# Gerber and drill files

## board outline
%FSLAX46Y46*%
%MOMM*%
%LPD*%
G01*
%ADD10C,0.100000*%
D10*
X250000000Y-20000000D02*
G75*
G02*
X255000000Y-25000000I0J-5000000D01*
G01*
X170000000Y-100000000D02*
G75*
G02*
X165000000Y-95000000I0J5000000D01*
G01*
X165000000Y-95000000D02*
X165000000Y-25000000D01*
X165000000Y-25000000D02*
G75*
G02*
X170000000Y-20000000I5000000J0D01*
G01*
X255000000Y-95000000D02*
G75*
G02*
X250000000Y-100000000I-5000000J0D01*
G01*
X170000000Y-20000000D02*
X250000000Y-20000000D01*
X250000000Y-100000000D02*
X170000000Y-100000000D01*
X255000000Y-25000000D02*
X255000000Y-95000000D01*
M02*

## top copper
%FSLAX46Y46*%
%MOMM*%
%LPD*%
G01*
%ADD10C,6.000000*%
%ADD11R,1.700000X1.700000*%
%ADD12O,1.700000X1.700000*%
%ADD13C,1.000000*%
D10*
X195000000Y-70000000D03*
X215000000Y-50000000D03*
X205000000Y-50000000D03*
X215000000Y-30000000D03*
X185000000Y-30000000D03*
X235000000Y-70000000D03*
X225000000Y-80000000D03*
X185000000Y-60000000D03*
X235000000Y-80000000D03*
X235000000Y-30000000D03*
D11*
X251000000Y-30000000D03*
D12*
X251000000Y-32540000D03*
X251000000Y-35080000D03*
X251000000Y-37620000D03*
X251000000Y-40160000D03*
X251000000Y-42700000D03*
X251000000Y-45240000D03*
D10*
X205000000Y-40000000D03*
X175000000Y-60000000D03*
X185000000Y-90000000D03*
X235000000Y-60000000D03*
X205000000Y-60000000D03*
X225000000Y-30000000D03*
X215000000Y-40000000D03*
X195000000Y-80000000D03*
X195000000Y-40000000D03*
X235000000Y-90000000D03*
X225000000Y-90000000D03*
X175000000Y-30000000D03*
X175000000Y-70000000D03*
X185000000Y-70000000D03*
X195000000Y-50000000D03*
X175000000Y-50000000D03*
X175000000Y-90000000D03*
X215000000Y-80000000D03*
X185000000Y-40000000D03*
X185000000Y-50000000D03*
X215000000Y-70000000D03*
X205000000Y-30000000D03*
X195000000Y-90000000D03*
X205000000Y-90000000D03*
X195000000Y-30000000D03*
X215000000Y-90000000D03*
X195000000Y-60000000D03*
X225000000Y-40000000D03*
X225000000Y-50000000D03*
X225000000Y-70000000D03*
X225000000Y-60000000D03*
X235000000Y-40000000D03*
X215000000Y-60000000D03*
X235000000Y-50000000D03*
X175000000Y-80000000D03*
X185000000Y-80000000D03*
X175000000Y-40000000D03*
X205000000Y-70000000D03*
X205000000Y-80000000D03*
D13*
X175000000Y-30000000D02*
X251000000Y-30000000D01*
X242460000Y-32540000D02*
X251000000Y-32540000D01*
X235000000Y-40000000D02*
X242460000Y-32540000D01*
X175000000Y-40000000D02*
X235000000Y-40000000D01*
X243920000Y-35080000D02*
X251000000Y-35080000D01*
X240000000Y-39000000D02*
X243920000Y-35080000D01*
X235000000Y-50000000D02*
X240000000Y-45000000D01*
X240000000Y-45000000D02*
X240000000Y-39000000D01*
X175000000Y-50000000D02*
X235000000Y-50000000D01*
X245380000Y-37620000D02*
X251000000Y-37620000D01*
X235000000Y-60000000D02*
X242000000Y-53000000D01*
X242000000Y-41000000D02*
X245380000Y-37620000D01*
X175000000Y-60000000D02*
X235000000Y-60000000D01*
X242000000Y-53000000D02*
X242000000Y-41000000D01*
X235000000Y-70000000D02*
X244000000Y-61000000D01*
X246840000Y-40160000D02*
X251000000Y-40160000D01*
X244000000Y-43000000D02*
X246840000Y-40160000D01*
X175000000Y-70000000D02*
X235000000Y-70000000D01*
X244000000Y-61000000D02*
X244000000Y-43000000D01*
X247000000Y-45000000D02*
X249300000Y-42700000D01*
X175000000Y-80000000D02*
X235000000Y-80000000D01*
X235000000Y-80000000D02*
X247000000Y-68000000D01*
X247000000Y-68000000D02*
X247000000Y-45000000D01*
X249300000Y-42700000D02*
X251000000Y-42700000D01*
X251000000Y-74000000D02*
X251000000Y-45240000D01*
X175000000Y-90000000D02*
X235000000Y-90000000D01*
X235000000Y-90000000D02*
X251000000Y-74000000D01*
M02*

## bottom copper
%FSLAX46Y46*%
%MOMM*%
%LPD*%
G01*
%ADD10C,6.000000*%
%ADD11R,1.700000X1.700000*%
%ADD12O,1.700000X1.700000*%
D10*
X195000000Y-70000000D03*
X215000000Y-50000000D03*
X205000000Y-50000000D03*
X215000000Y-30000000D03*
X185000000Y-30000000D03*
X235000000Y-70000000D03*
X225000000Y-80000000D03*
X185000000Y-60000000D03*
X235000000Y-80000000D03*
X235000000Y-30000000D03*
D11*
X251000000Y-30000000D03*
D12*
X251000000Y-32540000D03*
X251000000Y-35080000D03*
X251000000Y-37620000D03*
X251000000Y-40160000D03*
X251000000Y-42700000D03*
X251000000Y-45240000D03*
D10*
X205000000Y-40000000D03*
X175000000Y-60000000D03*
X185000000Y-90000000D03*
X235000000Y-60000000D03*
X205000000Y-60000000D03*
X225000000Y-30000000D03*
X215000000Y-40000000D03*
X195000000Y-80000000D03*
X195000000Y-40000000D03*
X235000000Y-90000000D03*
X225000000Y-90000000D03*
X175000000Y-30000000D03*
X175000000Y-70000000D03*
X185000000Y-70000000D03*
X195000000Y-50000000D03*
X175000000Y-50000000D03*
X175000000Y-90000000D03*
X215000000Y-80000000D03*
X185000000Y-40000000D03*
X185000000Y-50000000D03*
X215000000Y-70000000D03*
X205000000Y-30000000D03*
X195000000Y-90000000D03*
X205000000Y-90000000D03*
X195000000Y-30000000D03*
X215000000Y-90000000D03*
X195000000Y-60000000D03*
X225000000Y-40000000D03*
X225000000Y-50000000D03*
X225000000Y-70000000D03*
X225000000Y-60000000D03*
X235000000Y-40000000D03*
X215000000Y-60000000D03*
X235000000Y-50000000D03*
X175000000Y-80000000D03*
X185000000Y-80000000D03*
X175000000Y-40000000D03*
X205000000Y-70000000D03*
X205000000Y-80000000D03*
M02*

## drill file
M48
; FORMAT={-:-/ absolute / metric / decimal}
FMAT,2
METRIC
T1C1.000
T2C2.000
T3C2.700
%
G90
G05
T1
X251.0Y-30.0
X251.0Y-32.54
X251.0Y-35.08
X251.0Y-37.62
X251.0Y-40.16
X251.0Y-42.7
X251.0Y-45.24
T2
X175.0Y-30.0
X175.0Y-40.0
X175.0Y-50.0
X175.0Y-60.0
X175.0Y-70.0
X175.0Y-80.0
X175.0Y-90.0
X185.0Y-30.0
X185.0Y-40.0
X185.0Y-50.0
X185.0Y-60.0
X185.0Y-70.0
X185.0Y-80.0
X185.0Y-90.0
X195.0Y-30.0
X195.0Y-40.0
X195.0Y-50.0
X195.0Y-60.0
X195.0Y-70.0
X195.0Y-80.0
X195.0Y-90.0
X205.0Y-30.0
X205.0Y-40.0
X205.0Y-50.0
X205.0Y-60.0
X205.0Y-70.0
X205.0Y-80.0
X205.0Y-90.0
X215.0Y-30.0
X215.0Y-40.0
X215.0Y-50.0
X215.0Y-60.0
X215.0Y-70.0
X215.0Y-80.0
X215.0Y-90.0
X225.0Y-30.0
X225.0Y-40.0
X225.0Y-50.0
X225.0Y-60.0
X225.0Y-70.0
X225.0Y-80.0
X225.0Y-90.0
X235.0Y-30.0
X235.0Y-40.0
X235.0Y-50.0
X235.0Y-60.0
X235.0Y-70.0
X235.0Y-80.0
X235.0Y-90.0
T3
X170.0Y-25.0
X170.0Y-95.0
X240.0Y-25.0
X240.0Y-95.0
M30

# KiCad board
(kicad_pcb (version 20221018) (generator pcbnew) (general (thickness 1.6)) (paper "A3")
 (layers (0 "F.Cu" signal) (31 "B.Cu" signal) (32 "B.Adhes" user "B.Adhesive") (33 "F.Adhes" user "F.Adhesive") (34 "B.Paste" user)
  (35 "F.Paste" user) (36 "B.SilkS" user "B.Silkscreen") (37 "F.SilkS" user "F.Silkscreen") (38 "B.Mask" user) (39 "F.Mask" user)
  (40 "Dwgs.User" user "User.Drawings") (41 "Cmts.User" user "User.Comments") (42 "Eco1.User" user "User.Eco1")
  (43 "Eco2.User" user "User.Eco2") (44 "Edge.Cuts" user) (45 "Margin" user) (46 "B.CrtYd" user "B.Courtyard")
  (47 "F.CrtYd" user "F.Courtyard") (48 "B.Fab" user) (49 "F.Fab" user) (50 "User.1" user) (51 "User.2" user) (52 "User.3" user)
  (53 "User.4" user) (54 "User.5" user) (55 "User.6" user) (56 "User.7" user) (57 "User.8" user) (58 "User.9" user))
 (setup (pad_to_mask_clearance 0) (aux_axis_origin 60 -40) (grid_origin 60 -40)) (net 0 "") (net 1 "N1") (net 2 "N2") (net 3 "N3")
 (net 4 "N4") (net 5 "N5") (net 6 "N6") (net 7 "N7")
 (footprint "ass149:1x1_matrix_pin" (layer "F.Cu") (at 195 72.54)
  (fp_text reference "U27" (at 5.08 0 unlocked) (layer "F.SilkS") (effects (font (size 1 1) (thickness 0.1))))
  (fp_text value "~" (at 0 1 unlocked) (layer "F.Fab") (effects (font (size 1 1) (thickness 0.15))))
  (pad "1" thru_hole circle (at 0 -2.54) (size 6 6) (drill 2) (layers "*.Cu" "*.Mask") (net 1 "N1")))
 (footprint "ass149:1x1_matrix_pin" (layer "F.Cu") (at 215 47.46 180)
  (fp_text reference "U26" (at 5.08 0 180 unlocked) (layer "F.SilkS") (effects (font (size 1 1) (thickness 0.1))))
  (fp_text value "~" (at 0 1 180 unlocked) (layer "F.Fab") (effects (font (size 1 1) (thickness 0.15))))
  (pad "1" thru_hole circle (at 0 -2.54 180) (size 6 6) (drill 2) (layers "*.Cu" "*.Mask") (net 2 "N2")))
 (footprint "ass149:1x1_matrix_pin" (layer "F.Cu") (at 207.54 50 90)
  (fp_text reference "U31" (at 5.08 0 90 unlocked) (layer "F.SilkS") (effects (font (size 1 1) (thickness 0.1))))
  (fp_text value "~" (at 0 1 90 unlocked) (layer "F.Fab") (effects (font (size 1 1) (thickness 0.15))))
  (pad "1" thru_hole circle (at 0 -2.54 90) (size 6 6) (drill 2) (layers "*.Cu" "*.Mask") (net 2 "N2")))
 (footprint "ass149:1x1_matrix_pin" (layer "F.Cu") (at 217.54 30 90)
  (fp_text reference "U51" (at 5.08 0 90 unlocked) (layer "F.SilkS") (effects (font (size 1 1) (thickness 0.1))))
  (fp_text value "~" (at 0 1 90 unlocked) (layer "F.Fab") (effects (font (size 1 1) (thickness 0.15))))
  (pad "1" thru_hole circle (at 0 -2.54 90) (size 6 6) (drill 2) (layers "*.Cu" "*.Mask") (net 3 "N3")))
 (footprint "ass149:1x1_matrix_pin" (layer "F.Cu") (at 187.54 30 90)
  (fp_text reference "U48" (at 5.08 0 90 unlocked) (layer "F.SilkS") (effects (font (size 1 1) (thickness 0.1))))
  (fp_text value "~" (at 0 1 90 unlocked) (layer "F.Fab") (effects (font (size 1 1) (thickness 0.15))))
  (pad "1" thru_hole circle (at 0 -2.54 90) (size 6 6) (drill 2) (layers "*.Cu" "*.Mask") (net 3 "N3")))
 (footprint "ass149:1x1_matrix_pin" (layer "F.Cu") (at 232.46 70 -90)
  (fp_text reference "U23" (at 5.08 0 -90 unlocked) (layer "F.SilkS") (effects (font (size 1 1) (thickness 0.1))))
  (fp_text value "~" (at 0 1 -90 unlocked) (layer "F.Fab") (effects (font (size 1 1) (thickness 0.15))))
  (pad "1" thru_hole circle (at 0 -2.54 270) (size 6 6) (drill 2) (layers "*.Cu" "*.Mask") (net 1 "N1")))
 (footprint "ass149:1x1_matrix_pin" (layer "F.Cu") (at 227.54 80 90)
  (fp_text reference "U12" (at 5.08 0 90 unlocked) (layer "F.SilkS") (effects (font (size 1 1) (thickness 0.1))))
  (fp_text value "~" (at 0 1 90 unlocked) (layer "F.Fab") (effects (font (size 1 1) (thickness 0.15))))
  (pad "1" thru_hole circle (at 0 -2.54 90) (size 6 6) (drill 2) (layers "*.Cu" "*.Mask") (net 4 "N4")))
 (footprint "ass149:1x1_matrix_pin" (layer "F.Cu") (at 187.54 60 90)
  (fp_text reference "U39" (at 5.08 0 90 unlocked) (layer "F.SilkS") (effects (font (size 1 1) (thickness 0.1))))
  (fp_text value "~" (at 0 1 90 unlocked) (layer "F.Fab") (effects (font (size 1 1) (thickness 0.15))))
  (pad "1" thru_hole circle (at 0 -2.54 90) (size 6 6) (drill 2) (layers "*.Cu" "*.Mask") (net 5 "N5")))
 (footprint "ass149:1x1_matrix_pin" (layer "F.Cu") (at 235 77.46 180)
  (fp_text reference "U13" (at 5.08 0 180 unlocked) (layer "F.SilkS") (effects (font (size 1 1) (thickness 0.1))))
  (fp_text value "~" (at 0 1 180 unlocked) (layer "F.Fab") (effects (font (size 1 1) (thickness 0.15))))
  (pad "1" thru_hole circle (at 0 -2.54 180) (size 6 6) (drill 2) (layers "*.Cu" "*.Mask") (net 4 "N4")))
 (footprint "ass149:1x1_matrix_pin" (layer "F.Cu") (at 237.54 30 90)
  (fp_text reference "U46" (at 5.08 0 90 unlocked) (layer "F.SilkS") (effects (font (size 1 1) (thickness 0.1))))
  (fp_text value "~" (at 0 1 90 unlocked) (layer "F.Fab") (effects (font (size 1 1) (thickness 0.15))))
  (pad "1" thru_hole circle (at 0 -2.54 90) (size 6 6) (drill 2) (layers "*.Cu" "*.Mask") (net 3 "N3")))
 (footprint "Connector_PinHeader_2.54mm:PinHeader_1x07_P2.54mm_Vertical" (layer "F.Cu") (at 251 30)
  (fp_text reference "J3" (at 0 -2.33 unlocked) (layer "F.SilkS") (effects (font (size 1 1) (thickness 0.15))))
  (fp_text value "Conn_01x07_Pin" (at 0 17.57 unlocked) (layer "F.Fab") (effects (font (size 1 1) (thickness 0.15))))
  (pad "1" thru_hole rect (at 0 0) (size 1.7 1.7) (drill 1) (layers "*.Cu" "*.Mask") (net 3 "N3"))
  (pad "2" thru_hole oval (at 0 2.54) (size 1.7 1.7) (drill 1) (layers "*.Cu" "*.Mask") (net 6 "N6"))
  (pad "3" thru_hole oval (at 0 5.08) (size 1.7 1.7) (drill 1) (layers "*.Cu" "*.Mask") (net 2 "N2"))
  (pad "4" thru_hole oval (at 0 7.62) (size 1.7 1.7) (drill 1) (layers "*.Cu" "*.Mask") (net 5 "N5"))
  (pad "5" thru_hole oval (at 0 10.16) (size 1.7 1.7) (drill 1) (layers "*.Cu" "*.Mask") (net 1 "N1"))
  (pad "6" thru_hole oval (at 0 12.7) (size 1.7 1.7) (drill 1) (layers "*.Cu" "*.Mask") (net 4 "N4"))
  (pad "7" thru_hole oval (at 0 15.24) (size 1.7 1.7) (drill 1) (layers "*.Cu" "*.Mask") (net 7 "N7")))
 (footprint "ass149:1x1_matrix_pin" (layer "F.Cu") (at 207.54 40 90)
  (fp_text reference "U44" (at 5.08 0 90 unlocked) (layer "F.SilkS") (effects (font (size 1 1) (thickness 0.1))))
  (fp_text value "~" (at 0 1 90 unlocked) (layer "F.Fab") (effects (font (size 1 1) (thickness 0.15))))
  (pad "1" thru_hole circle (at 0 -2.54 90) (size 6 6) (drill 2) (layers "*.Cu" "*.Mask") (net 6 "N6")))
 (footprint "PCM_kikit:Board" (layer "F.Cu") (at 236.5 100 180)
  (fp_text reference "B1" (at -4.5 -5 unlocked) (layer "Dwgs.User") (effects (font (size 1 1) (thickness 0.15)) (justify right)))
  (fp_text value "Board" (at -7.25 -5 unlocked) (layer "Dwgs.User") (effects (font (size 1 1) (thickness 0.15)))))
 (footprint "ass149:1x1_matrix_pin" (layer "F.Cu") (at 175 57.46 180)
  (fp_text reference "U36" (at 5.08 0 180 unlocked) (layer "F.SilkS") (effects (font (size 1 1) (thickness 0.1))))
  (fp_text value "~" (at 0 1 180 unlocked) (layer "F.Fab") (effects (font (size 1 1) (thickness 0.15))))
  (pad "1" thru_hole circle (at 0 -2.54 180) (size 6 6) (drill 2) (layers "*.Cu" "*.Mask") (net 5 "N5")))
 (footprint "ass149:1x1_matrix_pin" (layer "F.Cu") (at 187.54 90 90)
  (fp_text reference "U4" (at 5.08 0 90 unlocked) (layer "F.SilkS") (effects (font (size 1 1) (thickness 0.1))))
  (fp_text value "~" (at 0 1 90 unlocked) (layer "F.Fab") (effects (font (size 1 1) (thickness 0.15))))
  (pad "1" thru_hole circle (at 0 -2.54 90) (size 6 6) (drill 2) (layers "*.Cu" "*.Mask") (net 7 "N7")))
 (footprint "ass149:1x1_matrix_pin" (layer "F.Cu") (at 235 57.46 180)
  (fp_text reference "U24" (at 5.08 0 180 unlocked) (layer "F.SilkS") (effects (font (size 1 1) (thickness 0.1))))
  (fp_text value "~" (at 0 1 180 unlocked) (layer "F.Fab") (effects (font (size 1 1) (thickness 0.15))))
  (pad "1" thru_hole circle (at 0 -2.54 180) (size 6 6) (drill 2) (layers "*.Cu" "*.Mask") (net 5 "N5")))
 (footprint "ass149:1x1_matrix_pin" (layer "F.Cu") (at 207.54 60 90)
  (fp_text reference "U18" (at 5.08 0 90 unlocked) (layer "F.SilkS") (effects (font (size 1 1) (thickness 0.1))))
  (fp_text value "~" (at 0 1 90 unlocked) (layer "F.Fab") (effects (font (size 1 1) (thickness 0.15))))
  (pad "1" thru_hole circle (at 0 -2.54 90) (size 6 6) (drill 2) (layers "*.Cu" "*.Mask") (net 5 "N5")))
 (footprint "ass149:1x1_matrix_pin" (layer "F.Cu") (at 225 32.54)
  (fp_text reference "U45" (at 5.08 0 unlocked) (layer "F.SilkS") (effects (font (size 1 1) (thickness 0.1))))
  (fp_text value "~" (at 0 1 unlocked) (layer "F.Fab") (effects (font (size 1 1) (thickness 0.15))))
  (pad "1" thru_hole circle (at 0 -2.54) (size 6 6) (drill 2) (layers "*.Cu" "*.Mask") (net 3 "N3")))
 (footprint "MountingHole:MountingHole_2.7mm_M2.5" (layer "F.Cu") (at 240 25)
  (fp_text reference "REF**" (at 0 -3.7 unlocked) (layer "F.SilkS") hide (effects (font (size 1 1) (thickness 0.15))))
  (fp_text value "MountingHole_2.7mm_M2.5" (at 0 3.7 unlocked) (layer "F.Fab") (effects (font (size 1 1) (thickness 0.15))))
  (pad "" np_thru_hole circle (at 0 0) (size 2.7 2.7) (drill 2.7) (layers "*.Cu" "*.Mask")))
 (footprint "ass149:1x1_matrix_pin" (layer "F.Cu") (at 217.54 40 90)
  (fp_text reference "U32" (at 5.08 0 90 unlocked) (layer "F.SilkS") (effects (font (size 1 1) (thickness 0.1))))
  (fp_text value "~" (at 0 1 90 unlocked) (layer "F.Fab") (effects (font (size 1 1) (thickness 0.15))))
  (pad "1" thru_hole circle (at 0 -2.54 90) (size 6 6) (drill 2) (layers "*.Cu" "*.Mask") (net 6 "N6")))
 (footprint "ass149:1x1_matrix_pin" (layer "F.Cu") (at 197.54 80 90)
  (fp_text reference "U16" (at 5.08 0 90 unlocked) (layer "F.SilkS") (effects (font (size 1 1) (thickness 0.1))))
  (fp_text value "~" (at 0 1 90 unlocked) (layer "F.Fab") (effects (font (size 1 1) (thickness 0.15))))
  (pad "1" thru_hole circle (at 0 -2.54 90) (size 6 6) (drill 2) (layers "*.Cu" "*.Mask") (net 4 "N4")))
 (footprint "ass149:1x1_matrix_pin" (layer "F.Cu") (at 197.54 40 90)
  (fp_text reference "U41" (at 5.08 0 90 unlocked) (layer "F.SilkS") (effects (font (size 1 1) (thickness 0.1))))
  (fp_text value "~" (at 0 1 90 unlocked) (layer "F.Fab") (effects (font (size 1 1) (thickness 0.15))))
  (pad "1" thru_hole circle (at 0 -2.54 90) (size 6 6) (drill 2) (layers "*.Cu" "*.Mask") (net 6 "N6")))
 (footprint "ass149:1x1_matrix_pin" (layer "F.Cu") (at 237.54 90 90)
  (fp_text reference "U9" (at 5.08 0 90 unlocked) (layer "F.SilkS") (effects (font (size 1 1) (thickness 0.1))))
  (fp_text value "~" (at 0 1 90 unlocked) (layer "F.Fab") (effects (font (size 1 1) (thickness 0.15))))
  (pad "1" thru_hole circle (at 0 -2.54 90) (size 6 6) (drill 2) (layers "*.Cu" "*.Mask") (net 7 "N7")))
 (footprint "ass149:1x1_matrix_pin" (layer "F.Cu") (at 227.54 90 90)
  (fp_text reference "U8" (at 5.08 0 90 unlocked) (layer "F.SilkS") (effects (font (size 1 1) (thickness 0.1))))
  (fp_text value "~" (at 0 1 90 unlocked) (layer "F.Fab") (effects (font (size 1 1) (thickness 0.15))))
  (pad "1" thru_hole circle (at 0 -2.54 90) (size 6 6) (drill 2) (layers "*.Cu" "*.Mask") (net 7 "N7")))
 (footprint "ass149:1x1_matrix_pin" (layer "F.Cu") (at 177.54 30 90)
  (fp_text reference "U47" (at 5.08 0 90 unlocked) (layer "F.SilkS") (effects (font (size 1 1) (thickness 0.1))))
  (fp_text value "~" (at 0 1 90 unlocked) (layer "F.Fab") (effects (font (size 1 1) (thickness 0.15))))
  (pad "1" thru_hole circle (at 0 -2.54 90) (size 6 6) (drill 2) (layers "*.Cu" "*.Mask") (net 3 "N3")))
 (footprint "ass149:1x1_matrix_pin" (layer "F.Cu") (at 177.54 70 90)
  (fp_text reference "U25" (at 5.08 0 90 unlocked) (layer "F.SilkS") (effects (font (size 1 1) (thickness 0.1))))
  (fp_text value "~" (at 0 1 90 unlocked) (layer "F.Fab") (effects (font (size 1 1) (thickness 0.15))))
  (pad "1" thru_hole circle (at 0 -2.54 90) (size 6 6) (drill 2) (layers "*.Cu" "*.Mask") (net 1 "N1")))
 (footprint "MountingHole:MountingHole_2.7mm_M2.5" (layer "F.Cu") (at 170 25)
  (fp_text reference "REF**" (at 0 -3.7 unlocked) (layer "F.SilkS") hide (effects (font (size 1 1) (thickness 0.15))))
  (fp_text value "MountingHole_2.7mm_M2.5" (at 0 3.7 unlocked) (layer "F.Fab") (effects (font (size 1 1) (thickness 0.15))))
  (pad "" np_thru_hole circle (at 0 0) (size 2.7 2.7) (drill 2.7) (layers "*.Cu" "*.Mask")))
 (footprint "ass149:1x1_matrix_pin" (layer "F.Cu") (at 187.54 70 90)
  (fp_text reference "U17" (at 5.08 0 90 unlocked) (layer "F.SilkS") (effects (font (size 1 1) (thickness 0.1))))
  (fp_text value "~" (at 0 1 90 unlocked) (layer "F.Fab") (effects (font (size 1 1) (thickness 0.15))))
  (pad "1" thru_hole circle (at 0 -2.54 90) (size 6 6) (drill 2) (layers "*.Cu" "*.Mask") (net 1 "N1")))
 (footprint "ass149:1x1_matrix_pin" (layer "F.Cu") (at 195 52.54)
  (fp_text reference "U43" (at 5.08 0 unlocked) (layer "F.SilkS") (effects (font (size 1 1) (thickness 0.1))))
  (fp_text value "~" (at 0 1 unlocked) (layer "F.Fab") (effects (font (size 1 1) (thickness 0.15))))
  (pad "1" thru_hole circle (at 0 -2.54) (size 6 6) (drill 2) (layers "*.Cu" "*.Mask") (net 2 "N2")))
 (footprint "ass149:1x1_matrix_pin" (layer "F.Cu") (at 177.54 50 90)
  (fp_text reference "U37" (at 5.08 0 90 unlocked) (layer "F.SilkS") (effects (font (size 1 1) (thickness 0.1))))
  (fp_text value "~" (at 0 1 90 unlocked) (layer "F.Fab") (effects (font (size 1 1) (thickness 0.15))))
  (pad "1" thru_hole circle (at 0 -2.54 90) (size 6 6) (drill 2) (layers "*.Cu" "*.Mask") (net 2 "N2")))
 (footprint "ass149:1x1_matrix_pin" (layer "F.Cu") (at 177.54 90 90)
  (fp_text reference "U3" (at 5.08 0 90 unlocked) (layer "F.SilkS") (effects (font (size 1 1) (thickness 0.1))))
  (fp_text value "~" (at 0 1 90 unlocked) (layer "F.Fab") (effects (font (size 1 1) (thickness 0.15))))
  (pad "1" thru_hole circle (at 0 -2.54 90) (size 6 6) (drill 2) (layers "*.Cu" "*.Mask") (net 7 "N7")))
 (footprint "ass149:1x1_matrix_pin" (layer "F.Cu") (at 217.54 80 90)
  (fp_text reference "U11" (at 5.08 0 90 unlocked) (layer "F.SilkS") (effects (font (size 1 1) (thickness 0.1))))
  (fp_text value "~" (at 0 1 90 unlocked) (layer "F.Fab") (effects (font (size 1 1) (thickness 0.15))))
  (pad "1" thru_hole circle (at 0 -2.54 90) (size 6 6) (drill 2) (layers "*.Cu" "*.Mask") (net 4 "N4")))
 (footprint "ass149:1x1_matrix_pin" (layer "F.Cu") (at 187.54 40 90)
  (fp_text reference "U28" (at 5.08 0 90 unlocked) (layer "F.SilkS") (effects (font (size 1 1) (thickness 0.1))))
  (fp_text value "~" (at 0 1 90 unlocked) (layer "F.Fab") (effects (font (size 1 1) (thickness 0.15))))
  (pad "1" thru_hole circle (at 0 -2.54 90) (size 6 6) (drill 2) (layers "*.Cu" "*.Mask") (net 6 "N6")))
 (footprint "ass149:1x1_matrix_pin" (layer "F.Cu") (at 187.54 50 90)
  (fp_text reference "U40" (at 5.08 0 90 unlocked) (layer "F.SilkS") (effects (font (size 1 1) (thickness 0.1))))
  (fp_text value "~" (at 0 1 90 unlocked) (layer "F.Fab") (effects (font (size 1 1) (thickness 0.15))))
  (pad "1" thru_hole circle (at 0 -2.54 90) (size 6 6) (drill 2) (layers "*.Cu" "*.Mask") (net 2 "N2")))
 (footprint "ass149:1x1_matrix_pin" (layer "F.Cu") (at 212.46 70 -90)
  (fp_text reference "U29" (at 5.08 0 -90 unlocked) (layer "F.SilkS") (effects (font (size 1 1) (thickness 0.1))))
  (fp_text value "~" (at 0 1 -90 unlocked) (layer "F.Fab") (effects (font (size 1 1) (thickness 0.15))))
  (pad "1" thru_hole circle (at 0 -2.54 270) (size 6 6) (drill 2) (layers "*.Cu" "*.Mask") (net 1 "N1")))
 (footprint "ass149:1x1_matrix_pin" (layer "F.Cu") (at 202.46 30 -90)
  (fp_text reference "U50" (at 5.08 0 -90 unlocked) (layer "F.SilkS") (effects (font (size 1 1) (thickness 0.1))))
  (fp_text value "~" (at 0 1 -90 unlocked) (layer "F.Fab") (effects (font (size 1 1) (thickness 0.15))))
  (pad "1" thru_hole circle (at 0 -2.54 270) (size 6 6) (drill 2) (layers "*.Cu" "*.Mask") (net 3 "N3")))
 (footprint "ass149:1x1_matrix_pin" (layer "F.Cu") (at 195 92.54)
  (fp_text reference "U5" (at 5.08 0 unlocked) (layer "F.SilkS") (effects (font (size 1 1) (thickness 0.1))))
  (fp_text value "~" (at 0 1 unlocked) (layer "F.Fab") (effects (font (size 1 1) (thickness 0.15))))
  (pad "1" thru_hole circle (at 0 -2.54) (size 6 6) (drill 2) (layers "*.Cu" "*.Mask") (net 7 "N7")))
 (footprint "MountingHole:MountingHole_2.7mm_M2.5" (layer "F.Cu") (at 240 95)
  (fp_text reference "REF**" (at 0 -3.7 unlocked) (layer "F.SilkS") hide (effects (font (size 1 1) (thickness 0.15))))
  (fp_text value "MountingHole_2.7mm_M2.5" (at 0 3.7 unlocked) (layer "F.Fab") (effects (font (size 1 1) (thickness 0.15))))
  (pad "" np_thru_hole circle (at 0 0) (size 2.7 2.7) (drill 2.7) (layers "*.Cu" "*.Mask")))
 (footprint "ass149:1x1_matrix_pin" (layer "F.Cu") (at 205 87.46 180)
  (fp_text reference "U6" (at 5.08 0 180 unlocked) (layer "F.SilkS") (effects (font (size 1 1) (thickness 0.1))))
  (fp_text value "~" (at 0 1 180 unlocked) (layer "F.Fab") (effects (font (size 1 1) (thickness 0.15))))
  (pad "1" thru_hole circle (at 0 -2.54 180) (size 6 6) (drill 2) (layers "*.Cu" "*.Mask") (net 7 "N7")))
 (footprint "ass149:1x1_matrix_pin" (layer "F.Cu") (at 197.54 30 90)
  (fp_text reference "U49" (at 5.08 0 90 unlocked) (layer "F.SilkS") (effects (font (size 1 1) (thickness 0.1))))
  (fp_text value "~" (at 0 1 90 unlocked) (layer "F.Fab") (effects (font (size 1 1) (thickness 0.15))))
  (pad "1" thru_hole circle (at 0 -2.54 90) (size 6 6) (drill 2) (layers "*.Cu" "*.Mask") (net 3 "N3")))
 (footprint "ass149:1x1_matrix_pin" (layer "F.Cu") (at 215 92.54)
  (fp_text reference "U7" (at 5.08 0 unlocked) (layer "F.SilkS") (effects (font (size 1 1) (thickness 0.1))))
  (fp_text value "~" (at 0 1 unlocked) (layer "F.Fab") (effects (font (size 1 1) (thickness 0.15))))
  (pad "1" thru_hole circle (at 0 -2.54) (size 6 6) (drill 2) (layers "*.Cu" "*.Mask") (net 7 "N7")))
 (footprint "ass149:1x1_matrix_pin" (layer "F.Cu") (at 195 62.54)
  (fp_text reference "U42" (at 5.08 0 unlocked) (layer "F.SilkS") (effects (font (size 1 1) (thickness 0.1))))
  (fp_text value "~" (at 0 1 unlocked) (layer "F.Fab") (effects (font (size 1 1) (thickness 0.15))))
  (pad "1" thru_hole circle (at 0 -2.54) (size 6 6) (drill 2) (layers "*.Cu" "*.Mask") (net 5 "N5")))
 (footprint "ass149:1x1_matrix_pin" (layer "F.Cu") (at 227.54 40 90)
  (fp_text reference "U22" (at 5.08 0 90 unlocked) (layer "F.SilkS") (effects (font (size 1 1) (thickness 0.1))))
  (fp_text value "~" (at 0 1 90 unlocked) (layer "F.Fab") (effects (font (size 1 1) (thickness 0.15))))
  (pad "1" thru_hole circle (at 0 -2.54 90) (size 6 6) (drill 2) (layers "*.Cu" "*.Mask") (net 6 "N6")))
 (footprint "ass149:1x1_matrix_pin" (layer "F.Cu") (at 222.46 50 -90)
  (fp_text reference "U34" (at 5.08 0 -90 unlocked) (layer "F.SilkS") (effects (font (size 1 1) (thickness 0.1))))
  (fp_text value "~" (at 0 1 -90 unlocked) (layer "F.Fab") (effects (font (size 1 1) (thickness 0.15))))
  (pad "1" thru_hole circle (at 0 -2.54 270) (size 6 6) (drill 2) (layers "*.Cu" "*.Mask") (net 2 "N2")))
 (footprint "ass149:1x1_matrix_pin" (layer "F.Cu") (at 225 72.54)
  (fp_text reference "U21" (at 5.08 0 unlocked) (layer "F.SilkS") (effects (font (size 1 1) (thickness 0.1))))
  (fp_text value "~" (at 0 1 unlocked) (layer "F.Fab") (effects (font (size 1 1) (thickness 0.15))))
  (pad "1" thru_hole circle (at 0 -2.54) (size 6 6) (drill 2) (layers "*.Cu" "*.Mask") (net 1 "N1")))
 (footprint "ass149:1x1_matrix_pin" (layer "F.Cu") (at 227.54 60 90)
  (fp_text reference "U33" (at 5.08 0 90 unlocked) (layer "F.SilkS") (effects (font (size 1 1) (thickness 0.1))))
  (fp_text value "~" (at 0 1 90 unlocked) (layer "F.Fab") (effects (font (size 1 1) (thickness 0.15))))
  (pad "1" thru_hole circle (at 0 -2.54 90) (size 6 6) (drill 2) (layers "*.Cu" "*.Mask") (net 5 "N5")))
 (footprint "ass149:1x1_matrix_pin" (layer "F.Cu") (at 235 37.46 180)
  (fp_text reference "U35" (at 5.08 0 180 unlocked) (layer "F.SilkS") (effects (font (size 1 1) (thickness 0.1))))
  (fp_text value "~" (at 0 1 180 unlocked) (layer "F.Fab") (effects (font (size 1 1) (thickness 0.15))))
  (pad "1" thru_hole circle (at 0 -2.54 180) (size 6 6) (drill 2) (layers "*.Cu" "*.Mask") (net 6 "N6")))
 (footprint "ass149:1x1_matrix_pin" (layer "F.Cu") (at 217.54 60 90)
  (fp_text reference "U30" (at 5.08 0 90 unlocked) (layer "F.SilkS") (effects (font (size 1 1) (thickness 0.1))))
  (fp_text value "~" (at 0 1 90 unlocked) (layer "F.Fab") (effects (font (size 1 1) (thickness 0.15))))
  (pad "1" thru_hole circle (at 0 -2.54 90) (size 6 6) (drill 2) (layers "*.Cu" "*.Mask") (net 5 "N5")))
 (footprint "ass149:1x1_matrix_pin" (layer "F.Cu") (at 232.46 50 -90)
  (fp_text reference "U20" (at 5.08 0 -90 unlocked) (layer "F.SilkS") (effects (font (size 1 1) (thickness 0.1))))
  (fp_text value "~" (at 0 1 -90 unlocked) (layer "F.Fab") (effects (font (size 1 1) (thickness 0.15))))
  (pad "1" thru_hole circle (at 0 -2.54 270) (size 6 6) (drill 2) (layers "*.Cu" "*.Mask") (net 2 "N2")))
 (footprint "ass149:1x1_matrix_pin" (layer "F.Cu") (at 175 77.46 180)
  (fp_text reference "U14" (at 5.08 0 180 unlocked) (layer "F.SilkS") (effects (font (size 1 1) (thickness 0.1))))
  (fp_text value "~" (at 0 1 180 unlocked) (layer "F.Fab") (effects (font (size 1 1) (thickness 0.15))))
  (pad "1" thru_hole circle (at 0 -2.54 180) (size 6 6) (drill 2) (layers "*.Cu" "*.Mask") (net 4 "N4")))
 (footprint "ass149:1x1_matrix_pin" (layer "F.Cu") (at 187.54 80 90)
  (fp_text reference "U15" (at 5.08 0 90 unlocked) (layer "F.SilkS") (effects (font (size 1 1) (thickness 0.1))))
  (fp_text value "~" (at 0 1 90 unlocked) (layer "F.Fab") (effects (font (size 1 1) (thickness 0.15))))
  (pad "1" thru_hole circle (at 0 -2.54 90) (size 6 6) (drill 2) (layers "*.Cu" "*.Mask") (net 4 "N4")))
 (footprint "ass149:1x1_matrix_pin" (layer "F.Cu") (at 172.46 40 -90)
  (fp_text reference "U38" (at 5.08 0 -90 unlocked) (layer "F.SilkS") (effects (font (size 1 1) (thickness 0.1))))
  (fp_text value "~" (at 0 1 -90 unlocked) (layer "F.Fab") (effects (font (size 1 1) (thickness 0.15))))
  (pad "1" thru_hole circle (at 0 -2.54 270) (size 6 6) (drill 2) (layers "*.Cu" "*.Mask") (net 6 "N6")))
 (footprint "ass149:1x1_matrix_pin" (layer "F.Cu") (at 207.54 70 90)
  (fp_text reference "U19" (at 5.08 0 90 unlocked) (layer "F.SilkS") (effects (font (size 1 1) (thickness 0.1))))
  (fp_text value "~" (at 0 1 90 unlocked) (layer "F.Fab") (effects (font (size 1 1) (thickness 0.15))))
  (pad "1" thru_hole circle (at 0 -2.54 90) (size 6 6) (drill 2) (layers "*.Cu" "*.Mask") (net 1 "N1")))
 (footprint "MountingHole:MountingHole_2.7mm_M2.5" (layer "F.Cu") (at 170 95)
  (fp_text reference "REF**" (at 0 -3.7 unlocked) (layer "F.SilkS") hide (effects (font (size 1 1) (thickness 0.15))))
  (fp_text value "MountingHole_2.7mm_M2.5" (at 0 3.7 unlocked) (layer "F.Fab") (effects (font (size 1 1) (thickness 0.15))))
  (pad "" np_thru_hole circle (at 0 0) (size 2.7 2.7) (drill 2.7) (layers "*.Cu" "*.Mask")))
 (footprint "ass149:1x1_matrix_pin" (layer "F.Cu") (at 202.46 80 -90)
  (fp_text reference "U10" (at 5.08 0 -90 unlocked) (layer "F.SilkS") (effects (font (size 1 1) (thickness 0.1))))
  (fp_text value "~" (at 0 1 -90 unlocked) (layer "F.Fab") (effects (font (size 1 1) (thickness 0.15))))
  (pad "1" thru_hole circle (at 0 -2.54 270) (size 6 6) (drill 2) (layers "*.Cu" "*.Mask") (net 4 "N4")))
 (gr_arc (start 250 20) (mid 253.535533 21.464466) (end 255 25) (stroke (width 0.1) (type default)) (layer "Edge.Cuts"))
 (gr_arc (start 170 100) (mid 166.464466 98.535533) (end 165 95) (stroke (width 0.1) (type default)) (layer "Edge.Cuts"))
 (gr_line (start 165 95) (end 165 25) (stroke (width 0.1) (type default)) (layer "Edge.Cuts"))
 (gr_arc (start 165 25) (mid 166.464466 21.464466) (end 170 20) (stroke (width 0.1) (type default)) (layer "Edge.Cuts"))
 (gr_arc (start 255 95) (mid 253.535533 98.535533) (end 250 100) (stroke (width 0.1) (type default)) (layer "Edge.Cuts"))
 (gr_line (start 170 20) (end 250 20) (stroke (width 0.1) (type default)) (layer "Edge.Cuts"))
 (gr_line (start 250 100) (end 170 100) (stroke (width 0.1) (type default)) (layer "Edge.Cuts"))
 (gr_line (start 255 25) (end 255 95) (stroke (width 0.1) (type default)) (layer "Edge.Cuts"))
 (segment (start 175 30) (end 251 30) (width 1) (layer "F.Cu") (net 3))
 (segment (start 242.46 32.54) (end 251 32.54) (width 1) (layer "F.Cu") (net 6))
 (segment (start 235 40) (end 242.46 32.54) (width 1) (layer "F.Cu") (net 6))
 (segment (start 175 40) (end 235 40) (width 1) (layer "F.Cu") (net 6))
 (segment (start 243.92 35.08) (end 251 35.08) (width 1) (layer "F.Cu") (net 2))
 (segment (start 240 39) (end 243.92 35.08) (width 1) (layer "F.Cu") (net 2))
 (segment (start 235 50) (end 240 45) (width 1) (layer "F.Cu") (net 2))
 (segment (start 240 45) (end 240 39) (width 1) (layer "F.Cu") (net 2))
 (segment (start 175 50) (end 235 50) (width 1) (layer "F.Cu") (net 2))
 (segment (start 245.38 37.62) (end 251 37.62) (width 1) (layer "F.Cu") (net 5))
 (segment (start 235 60) (end 242 53) (width 1) (layer "F.Cu") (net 5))
 (segment (start 242 41) (end 245.38 37.62) (width 1) (layer "F.Cu") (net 5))
 (segment (start 175 60) (end 235 60) (width 1) (layer "F.Cu") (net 5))
 (segment (start 242 53) (end 242 41) (width 1) (layer "F.Cu") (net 5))
 (segment (start 235 70) (end 244 61) (width 1) (layer "F.Cu") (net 1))
 (segment (start 246.84 40.16) (end 251 40.16) (width 1) (layer "F.Cu") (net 1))
 (segment (start 244 43) (end 246.84 40.16) (width 1) (layer "F.Cu") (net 1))
 (segment (start 175 70) (end 235 70) (width 1) (layer "F.Cu") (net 1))
 (segment (start 244 61) (end 244 43) (width 1) (layer "F.Cu") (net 1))
 (segment (start 247 45) (end 249.3 42.7) (width 1) (layer "F.Cu") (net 4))
 (segment (start 175 80) (end 235 80) (width 1) (layer "F.Cu") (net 4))
 (segment (start 235 80) (end 247 68) (width 1) (layer "F.Cu") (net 4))
 (segment (start 247 68) (end 247 45) (width 1) (layer "F.Cu") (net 4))
 (segment (start 249.3 42.7) (end 251 42.7) (width 1) (layer "F.Cu") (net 4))
 (segment (start 251 74) (end 251 45.24) (width 1) (layer "F.Cu") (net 7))
 (segment (start 175 90) (end 235 90) (width 1) (layer "F.Cu") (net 7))
 (segment (start 235 90) (end 251 74) (width 1) (layer "F.Cu") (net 7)))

